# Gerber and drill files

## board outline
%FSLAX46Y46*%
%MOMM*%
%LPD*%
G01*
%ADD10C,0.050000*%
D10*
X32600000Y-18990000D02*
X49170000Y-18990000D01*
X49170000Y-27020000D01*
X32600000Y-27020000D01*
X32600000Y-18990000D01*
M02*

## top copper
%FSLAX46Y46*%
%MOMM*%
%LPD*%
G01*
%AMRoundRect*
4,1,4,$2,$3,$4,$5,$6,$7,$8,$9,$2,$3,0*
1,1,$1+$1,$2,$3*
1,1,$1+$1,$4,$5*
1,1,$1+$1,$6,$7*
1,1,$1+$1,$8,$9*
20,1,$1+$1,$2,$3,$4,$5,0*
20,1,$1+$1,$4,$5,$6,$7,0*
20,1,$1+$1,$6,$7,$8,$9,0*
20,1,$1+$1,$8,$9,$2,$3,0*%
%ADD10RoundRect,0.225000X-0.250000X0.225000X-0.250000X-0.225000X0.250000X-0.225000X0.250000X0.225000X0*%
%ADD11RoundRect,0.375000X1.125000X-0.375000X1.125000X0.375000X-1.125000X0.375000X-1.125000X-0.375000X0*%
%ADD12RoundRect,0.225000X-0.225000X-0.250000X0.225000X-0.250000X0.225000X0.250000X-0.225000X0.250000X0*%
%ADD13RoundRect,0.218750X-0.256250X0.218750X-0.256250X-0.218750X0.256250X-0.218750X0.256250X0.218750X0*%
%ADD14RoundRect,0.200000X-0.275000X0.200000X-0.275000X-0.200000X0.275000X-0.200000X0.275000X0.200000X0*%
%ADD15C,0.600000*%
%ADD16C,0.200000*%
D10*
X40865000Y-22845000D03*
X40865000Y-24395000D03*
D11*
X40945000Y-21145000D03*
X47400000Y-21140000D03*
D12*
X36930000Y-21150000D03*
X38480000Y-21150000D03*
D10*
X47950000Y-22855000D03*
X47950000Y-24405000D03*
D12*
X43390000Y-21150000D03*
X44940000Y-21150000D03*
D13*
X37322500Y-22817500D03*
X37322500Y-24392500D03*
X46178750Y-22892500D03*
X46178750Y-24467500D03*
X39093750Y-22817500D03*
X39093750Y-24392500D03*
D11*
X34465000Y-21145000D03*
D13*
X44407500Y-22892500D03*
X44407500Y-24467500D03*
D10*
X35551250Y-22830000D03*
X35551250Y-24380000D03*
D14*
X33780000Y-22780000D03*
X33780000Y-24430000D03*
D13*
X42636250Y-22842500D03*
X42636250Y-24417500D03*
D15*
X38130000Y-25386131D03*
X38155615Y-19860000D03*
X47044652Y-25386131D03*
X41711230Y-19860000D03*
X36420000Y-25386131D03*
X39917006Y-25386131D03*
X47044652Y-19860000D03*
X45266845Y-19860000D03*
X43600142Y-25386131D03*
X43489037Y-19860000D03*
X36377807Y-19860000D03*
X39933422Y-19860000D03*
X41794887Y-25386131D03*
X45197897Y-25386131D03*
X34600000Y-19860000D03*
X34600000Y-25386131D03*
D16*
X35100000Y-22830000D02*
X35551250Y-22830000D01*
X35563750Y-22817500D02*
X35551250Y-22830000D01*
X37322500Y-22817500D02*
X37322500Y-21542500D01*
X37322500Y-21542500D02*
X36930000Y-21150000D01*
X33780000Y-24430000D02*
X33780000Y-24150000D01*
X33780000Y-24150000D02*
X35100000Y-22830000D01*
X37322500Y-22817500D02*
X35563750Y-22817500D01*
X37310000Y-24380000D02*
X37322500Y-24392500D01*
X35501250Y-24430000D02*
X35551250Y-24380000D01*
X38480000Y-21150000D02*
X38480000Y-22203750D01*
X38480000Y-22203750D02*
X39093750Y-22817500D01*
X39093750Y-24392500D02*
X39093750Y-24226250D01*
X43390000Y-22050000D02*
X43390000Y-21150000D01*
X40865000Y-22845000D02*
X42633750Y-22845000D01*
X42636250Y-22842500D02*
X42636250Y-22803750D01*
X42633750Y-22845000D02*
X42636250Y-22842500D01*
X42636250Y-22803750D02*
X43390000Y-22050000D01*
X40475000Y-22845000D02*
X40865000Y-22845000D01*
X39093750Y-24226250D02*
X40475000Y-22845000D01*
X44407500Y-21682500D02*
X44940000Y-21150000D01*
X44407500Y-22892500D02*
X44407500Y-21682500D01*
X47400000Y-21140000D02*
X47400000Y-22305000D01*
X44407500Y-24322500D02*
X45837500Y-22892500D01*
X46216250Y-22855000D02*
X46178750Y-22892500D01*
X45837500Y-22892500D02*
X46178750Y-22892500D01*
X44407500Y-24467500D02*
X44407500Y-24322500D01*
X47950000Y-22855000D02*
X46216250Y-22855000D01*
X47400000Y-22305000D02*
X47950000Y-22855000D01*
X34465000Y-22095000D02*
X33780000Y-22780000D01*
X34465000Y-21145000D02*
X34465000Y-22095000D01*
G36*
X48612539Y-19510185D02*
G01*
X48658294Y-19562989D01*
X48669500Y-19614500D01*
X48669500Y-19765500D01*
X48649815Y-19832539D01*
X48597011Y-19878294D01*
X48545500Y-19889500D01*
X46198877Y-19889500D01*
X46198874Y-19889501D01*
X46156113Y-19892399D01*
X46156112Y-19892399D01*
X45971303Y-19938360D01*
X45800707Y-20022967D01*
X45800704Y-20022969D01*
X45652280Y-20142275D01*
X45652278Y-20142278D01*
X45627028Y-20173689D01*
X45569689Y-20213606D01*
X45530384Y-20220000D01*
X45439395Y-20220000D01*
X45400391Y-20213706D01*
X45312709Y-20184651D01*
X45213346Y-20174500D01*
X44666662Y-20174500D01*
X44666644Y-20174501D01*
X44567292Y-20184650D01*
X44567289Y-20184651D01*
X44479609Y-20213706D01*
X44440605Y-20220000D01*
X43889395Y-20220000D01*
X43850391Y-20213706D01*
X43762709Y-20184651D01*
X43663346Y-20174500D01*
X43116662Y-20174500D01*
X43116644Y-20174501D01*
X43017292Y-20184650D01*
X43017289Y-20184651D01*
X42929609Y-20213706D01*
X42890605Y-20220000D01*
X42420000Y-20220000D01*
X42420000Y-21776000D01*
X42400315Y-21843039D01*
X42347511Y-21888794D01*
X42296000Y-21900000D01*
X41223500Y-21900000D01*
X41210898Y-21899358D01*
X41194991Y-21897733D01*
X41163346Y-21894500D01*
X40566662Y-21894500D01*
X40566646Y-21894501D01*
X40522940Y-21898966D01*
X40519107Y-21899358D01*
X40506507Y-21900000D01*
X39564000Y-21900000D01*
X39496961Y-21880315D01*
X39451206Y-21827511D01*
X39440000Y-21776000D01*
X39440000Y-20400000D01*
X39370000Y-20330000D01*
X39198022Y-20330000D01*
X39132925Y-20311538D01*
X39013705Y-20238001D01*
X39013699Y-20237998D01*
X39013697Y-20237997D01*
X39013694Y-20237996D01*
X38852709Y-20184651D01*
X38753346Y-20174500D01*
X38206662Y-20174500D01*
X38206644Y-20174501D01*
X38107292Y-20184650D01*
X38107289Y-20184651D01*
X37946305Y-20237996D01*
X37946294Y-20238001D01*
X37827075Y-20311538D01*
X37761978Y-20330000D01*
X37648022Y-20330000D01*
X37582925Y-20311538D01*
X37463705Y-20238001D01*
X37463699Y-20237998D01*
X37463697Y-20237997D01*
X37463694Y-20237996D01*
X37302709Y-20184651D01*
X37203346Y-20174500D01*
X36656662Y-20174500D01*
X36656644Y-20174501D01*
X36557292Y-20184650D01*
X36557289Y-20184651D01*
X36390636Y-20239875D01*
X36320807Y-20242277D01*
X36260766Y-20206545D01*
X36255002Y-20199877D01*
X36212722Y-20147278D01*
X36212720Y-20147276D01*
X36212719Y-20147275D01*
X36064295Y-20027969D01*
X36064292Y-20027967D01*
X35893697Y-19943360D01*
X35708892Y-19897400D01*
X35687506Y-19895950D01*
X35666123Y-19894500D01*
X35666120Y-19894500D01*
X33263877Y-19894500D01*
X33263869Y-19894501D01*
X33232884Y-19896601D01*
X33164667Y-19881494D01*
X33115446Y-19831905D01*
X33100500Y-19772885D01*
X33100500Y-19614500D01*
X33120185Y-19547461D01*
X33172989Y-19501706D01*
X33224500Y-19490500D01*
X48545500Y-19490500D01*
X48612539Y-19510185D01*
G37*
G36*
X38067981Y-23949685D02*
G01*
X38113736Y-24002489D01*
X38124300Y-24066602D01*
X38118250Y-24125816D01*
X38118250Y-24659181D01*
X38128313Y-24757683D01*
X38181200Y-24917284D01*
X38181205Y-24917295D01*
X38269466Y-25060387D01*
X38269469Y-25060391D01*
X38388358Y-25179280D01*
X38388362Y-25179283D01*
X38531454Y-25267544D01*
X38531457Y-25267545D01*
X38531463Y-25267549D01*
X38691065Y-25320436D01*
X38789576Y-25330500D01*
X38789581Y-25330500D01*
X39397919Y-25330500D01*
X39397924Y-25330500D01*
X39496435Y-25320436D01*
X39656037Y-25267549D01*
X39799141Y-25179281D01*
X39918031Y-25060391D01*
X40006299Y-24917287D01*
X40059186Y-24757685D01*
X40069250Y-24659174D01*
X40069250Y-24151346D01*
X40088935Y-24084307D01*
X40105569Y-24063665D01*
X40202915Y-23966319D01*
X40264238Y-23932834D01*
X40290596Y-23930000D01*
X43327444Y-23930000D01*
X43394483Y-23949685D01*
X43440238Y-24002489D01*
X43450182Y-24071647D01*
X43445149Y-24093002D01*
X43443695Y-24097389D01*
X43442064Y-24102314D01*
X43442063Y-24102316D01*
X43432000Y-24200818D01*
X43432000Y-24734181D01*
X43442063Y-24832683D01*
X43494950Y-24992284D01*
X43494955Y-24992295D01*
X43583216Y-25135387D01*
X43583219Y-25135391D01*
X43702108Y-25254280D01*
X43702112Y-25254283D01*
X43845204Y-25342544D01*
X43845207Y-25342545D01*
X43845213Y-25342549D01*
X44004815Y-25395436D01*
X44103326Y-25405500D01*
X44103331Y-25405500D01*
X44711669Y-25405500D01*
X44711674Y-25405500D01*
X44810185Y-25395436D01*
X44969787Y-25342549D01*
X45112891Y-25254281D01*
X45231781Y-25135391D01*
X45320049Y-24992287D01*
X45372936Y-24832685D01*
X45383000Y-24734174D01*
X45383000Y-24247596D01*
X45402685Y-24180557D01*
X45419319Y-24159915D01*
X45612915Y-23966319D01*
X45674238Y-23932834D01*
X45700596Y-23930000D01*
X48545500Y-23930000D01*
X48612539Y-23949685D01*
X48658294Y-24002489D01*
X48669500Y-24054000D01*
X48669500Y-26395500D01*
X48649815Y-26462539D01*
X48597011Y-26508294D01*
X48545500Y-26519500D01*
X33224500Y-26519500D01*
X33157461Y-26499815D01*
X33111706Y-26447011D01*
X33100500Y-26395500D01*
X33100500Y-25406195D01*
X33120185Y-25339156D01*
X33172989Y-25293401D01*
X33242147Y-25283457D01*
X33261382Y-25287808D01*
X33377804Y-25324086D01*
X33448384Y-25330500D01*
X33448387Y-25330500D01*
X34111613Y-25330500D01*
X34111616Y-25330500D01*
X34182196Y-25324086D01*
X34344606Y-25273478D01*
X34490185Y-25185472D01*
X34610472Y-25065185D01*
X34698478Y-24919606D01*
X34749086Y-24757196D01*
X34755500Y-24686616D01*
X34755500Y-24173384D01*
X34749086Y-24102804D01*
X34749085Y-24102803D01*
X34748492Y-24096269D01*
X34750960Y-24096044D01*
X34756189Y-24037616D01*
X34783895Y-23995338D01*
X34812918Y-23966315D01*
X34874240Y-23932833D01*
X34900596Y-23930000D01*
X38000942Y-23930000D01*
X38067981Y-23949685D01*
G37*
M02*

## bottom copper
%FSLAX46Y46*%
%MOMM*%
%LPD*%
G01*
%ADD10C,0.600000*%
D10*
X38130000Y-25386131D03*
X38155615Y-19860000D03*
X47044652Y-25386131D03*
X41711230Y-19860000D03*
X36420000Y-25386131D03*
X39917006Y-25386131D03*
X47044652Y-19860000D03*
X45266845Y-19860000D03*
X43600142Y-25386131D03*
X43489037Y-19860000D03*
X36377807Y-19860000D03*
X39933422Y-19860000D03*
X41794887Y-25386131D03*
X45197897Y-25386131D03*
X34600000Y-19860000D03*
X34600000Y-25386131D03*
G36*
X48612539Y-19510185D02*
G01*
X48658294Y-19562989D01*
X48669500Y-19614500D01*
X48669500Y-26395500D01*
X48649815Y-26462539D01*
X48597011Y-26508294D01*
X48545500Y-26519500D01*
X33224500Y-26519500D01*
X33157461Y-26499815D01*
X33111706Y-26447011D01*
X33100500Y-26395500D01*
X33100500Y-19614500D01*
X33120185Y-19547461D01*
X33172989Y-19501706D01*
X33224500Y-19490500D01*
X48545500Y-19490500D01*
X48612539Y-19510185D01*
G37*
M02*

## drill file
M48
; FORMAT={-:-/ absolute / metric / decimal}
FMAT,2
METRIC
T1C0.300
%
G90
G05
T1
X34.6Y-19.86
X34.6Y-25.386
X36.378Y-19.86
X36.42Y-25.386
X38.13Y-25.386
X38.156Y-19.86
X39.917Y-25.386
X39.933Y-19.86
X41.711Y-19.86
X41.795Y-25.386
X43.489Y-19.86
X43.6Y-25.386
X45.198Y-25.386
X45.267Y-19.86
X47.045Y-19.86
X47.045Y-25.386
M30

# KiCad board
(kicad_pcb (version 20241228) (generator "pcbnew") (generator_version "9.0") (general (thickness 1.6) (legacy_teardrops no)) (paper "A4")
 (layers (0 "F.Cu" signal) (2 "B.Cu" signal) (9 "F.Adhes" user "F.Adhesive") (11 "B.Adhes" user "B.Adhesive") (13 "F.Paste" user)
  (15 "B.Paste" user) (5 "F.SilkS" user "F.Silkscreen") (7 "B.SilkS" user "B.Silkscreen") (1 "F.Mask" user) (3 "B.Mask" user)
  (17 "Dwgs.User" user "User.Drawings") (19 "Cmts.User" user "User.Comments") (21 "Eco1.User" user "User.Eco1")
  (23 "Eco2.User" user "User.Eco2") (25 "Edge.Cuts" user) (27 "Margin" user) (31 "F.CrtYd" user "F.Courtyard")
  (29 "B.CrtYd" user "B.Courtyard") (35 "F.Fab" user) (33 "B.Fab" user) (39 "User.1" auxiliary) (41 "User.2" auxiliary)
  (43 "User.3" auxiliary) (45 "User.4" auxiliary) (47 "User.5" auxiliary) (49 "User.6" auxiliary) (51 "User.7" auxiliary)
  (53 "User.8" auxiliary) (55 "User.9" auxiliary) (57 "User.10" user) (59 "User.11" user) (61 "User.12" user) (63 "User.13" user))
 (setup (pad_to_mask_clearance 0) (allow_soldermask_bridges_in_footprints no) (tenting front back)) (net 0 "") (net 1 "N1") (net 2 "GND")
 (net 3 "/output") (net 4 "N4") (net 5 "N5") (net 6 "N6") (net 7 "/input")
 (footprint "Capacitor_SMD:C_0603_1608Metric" (layer "F.Cu") (at 40.865 23.62 -90)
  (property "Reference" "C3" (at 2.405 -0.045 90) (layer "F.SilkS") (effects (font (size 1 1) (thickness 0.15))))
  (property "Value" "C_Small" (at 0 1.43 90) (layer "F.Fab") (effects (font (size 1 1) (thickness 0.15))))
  (pad "1" smd roundrect (at -0.775 0 270) (size 0.9 0.95) (layers "F.Cu" "F.Mask" "F.Paste") (roundrect_rratio 0.25) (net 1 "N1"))
  (pad "2" smd roundrect (at 0.775 0 270) (size 0.9 0.95) (layers "F.Cu" "F.Mask" "F.Paste") (roundrect_rratio 0.25) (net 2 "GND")))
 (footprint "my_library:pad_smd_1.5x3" (layer "F.Cu") (at 40.945 21.145)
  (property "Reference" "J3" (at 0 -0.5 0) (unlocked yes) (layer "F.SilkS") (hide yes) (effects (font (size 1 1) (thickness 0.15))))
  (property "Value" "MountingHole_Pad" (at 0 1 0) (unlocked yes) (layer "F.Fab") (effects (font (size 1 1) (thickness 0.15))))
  (pad "1" smd roundrect (at 0 0 90) (size 1.5 3) (layers "F.Cu" "F.Mask" "F.Paste") (roundrect_rratio 0.25) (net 2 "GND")
   (thermal_bridge_angle 45)))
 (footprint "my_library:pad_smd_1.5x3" (layer "F.Cu") (at 47.4 21.14)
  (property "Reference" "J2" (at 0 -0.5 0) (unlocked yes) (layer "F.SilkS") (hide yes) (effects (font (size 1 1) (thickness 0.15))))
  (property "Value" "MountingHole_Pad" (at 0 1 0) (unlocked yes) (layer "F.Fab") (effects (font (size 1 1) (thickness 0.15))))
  (pad "1" smd roundrect (at 0 0 90) (size 1.5 3) (layers "F.Cu" "F.Mask" "F.Paste") (roundrect_rratio 0.25) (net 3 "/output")
   (thermal_bridge_angle 45)))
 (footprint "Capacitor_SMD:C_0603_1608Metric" (layer "F.Cu") (at 37.705 21.15)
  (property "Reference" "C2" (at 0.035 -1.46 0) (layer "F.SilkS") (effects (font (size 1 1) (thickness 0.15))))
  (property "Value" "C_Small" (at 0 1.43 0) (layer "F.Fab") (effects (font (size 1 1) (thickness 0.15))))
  (pad "1" smd roundrect (at -0.775 0) (size 0.9 0.95) (layers "F.Cu" "F.Mask" "F.Paste") (roundrect_rratio 0.25) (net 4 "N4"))
  (pad "2" smd roundrect (at 0.775 0) (size 0.9 0.95) (layers "F.Cu" "F.Mask" "F.Paste") (roundrect_rratio 0.25) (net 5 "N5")))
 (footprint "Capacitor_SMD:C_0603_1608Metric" (layer "F.Cu") (at 47.95 23.63 -90)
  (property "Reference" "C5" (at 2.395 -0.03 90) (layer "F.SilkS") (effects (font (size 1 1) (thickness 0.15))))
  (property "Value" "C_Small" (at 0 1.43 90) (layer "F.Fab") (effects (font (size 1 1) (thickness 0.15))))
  (pad "1" smd roundrect (at -0.775 0 270) (size 0.9 0.95) (layers "F.Cu" "F.Mask" "F.Paste") (roundrect_rratio 0.25) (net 3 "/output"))
  (pad "2" smd roundrect (at 0.775 0 270) (size 0.9 0.95) (layers "F.Cu" "F.Mask" "F.Paste") (roundrect_rratio 0.25) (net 2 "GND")))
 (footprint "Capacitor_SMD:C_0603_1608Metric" (layer "F.Cu") (at 44.165 21.15)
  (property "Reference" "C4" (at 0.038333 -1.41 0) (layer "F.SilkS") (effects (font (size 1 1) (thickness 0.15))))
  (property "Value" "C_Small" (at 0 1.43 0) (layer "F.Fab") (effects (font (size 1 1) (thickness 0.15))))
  (pad "1" smd roundrect (at -0.775 0) (size 0.9 0.95) (layers "F.Cu" "F.Mask" "F.Paste") (roundrect_rratio 0.25) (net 1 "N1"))
  (pad "2" smd roundrect (at 0.775 0) (size 0.9 0.95) (layers "F.Cu" "F.Mask" "F.Paste") (roundrect_rratio 0.25) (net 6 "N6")))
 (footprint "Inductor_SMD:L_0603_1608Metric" (layer "F.Cu") (at 37.3225 23.605 -90)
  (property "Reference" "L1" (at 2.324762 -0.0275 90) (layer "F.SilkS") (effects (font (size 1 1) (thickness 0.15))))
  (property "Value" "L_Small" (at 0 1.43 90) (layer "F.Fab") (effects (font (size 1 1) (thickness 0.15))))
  (pad "1" smd roundrect (at -0.7875 0 270) (size 0.875 0.95) (layers "F.Cu" "F.Mask" "F.Paste") (roundrect_rratio 0.25) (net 4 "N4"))
  (pad "2" smd roundrect (at 0.7875 0 270) (size 0.875 0.95) (layers "F.Cu" "F.Mask" "F.Paste") (roundrect_rratio 0.25) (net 2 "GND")))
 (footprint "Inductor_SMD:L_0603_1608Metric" (layer "F.Cu") (at 46.17875 23.68 -90)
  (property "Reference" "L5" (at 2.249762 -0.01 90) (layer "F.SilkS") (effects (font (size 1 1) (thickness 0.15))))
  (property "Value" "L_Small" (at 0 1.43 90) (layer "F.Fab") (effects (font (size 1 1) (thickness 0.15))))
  (pad "1" smd roundrect (at -0.7875 0 270) (size 0.875 0.95) (layers "F.Cu" "F.Mask" "F.Paste") (roundrect_rratio 0.25) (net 3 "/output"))
  (pad "2" smd roundrect (at 0.7875 0 270) (size 0.875 0.95) (layers "F.Cu" "F.Mask" "F.Paste") (roundrect_rratio 0.25) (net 2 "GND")))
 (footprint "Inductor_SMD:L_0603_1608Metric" (layer "F.Cu") (at 39.09375 23.605 -90)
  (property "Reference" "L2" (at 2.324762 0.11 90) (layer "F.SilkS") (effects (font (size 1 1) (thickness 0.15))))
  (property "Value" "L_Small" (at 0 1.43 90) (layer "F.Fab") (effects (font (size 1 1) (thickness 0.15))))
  (pad "1" smd roundrect (at -0.7875 0 270) (size 0.875 0.95) (layers "F.Cu" "F.Mask" "F.Paste") (roundrect_rratio 0.25) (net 5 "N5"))
  (pad "2" smd roundrect (at 0.7875 0 270) (size 0.875 0.95) (layers "F.Cu" "F.Mask" "F.Paste") (roundrect_rratio 0.25) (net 1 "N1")))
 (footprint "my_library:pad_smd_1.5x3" (layer "F.Cu") (at 34.465 21.145)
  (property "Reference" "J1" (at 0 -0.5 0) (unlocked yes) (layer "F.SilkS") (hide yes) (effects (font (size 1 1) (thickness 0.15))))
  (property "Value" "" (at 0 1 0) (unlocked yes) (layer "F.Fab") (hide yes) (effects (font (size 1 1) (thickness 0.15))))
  (pad "1" smd roundrect (at 0 0 90) (size 1.5 3) (layers "F.Cu" "F.Mask" "F.Paste") (roundrect_rratio 0.25) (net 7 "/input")
   (thermal_bridge_angle 45)))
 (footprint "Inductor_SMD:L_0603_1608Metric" (layer "F.Cu") (at 44.4075 23.68 -90)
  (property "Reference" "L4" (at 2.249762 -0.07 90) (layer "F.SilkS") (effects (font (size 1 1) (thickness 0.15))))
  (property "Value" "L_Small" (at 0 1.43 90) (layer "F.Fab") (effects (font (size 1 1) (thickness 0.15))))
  (pad "1" smd roundrect (at -0.7875 0 270) (size 0.875 0.95) (layers "F.Cu" "F.Mask" "F.Paste") (roundrect_rratio 0.25) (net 6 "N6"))
  (pad "2" smd roundrect (at 0.7875 0 270) (size 0.875 0.95) (layers "F.Cu" "F.Mask" "F.Paste") (roundrect_rratio 0.25) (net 3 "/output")))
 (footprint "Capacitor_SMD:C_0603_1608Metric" (layer "F.Cu") (at 35.55125 23.605 -90)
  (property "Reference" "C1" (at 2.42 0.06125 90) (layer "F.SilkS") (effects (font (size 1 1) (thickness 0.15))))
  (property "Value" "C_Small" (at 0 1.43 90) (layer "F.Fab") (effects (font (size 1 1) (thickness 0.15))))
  (pad "1" smd roundrect (at -0.775 0 270) (size 0.9 0.95) (layers "F.Cu" "F.Mask" "F.Paste") (roundrect_rratio 0.25) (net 4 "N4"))
  (pad "2" smd roundrect (at 0.775 0 270) (size 0.9 0.95) (layers "F.Cu" "F.Mask" "F.Paste") (roundrect_rratio 0.25) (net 2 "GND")))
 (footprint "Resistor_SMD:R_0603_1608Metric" (layer "F.Cu") (at 33.78 23.605 -90)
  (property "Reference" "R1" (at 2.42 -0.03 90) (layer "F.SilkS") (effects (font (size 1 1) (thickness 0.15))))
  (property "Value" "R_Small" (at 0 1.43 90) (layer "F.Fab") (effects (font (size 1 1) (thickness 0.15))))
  (pad "1" smd roundrect (at -0.825 0 270) (size 0.8 0.95) (layers "F.Cu" "F.Mask" "F.Paste") (roundrect_rratio 0.25) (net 7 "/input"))
  (pad "2" smd roundrect (at 0.825 0 270) (size 0.8 0.95) (layers "F.Cu" "F.Mask" "F.Paste") (roundrect_rratio 0.25) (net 4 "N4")))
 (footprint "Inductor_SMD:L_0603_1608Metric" (layer "F.Cu") (at 42.63625 23.63 -90)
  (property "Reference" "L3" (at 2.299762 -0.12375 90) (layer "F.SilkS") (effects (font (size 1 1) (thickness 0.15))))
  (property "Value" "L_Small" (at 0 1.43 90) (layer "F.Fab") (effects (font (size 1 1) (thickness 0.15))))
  (pad "1" smd roundrect (at -0.7875 0 270) (size 0.875 0.95) (layers "F.Cu" "F.Mask" "F.Paste") (roundrect_rratio 0.25) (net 1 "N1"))
  (pad "2" smd roundrect (at 0.7875 0 270) (size 0.875 0.95) (layers "F.Cu" "F.Mask" "F.Paste") (roundrect_rratio 0.25) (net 2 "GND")))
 (gr_rect (start 32.6 18.99) (end 49.17 27.02) (stroke (width 0.05) (type default)) (fill no) (layer "Edge.Cuts"))
 (segment (start 35.1 22.83) (end 35.55125 22.83) (width 0.2) (layer "F.Cu") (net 4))
 (segment (start 35.56375 22.8175) (end 35.55125 22.83) (width 0.2) (layer "F.Cu") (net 4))
 (segment (start 37.3225 22.8175) (end 37.3225 21.5425) (width 0.2) (layer "F.Cu") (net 4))
 (segment (start 37.3225 21.5425) (end 36.93 21.15) (width 0.2) (layer "F.Cu") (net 4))
 (segment (start 33.78 24.43) (end 33.78 24.15) (width 0.2) (layer "F.Cu") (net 4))
 (segment (start 33.78 24.15) (end 35.1 22.83) (width 0.2) (layer "F.Cu") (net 4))
 (segment (start 37.3225 22.8175) (end 35.56375 22.8175) (width 0.2) (layer "F.Cu") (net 4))
 (segment (start 37.31 24.38) (end 37.3225 24.3925) (width 0.2) (layer "F.Cu") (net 2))
 (segment (start 35.50125 24.43) (end 35.55125 24.38) (width 0.2) (layer "F.Cu") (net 2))
 (via (at 38.13 25.386131) (size 0.6) (drill 0.3) (layers "F.Cu" "B.Cu") (free yes) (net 2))
 (via (at 38.155615 19.86) (size 0.6) (drill 0.3) (layers "F.Cu" "B.Cu") (free yes) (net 2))
 (via (at 47.044652 25.386131) (size 0.6) (drill 0.3) (layers "F.Cu" "B.Cu") (free yes) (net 2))
 (via (at 41.71123 19.86) (size 0.6) (drill 0.3) (layers "F.Cu" "B.Cu") (free yes) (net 2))
 (via (at 36.42 25.386131) (size 0.6) (drill 0.3) (layers "F.Cu" "B.Cu") (free yes) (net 2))
 (via (at 39.917006 25.386131) (size 0.6) (drill 0.3) (layers "F.Cu" "B.Cu") (free yes) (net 2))
 (via (at 47.044652 19.86) (size 0.6) (drill 0.3) (layers "F.Cu" "B.Cu") (free yes) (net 2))
 (via (at 45.266845 19.86) (size 0.6) (drill 0.3) (layers "F.Cu" "B.Cu") (free yes) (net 2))
 (via (at 43.600142 25.386131) (size 0.6) (drill 0.3) (layers "F.Cu" "B.Cu") (free yes) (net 2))
 (via (at 43.489037 19.86) (size 0.6) (drill 0.3) (layers "F.Cu" "B.Cu") (free yes) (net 2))
 (via (at 36.377807 19.86) (size 0.6) (drill 0.3) (layers "F.Cu" "B.Cu") (free yes) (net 2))
 (via (at 39.933422 19.86) (size 0.6) (drill 0.3) (layers "F.Cu" "B.Cu") (free yes) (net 2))
 (via (at 41.794887 25.386131) (size 0.6) (drill 0.3) (layers "F.Cu" "B.Cu") (free yes) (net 2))
 (via (at 45.197897 25.386131) (size 0.6) (drill 0.3) (layers "F.Cu" "B.Cu") (free yes) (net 2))
 (via (at 34.6 19.86) (size 0.6) (drill 0.3) (layers "F.Cu" "B.Cu") (free yes) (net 2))
 (via (at 34.6 25.386131) (size 0.6) (drill 0.3) (layers "F.Cu" "B.Cu") (free yes) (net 2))
 (segment (start 38.48 21.15) (end 38.48 22.20375) (width 0.2) (layer "F.Cu") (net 5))
 (segment (start 38.48 22.20375) (end 39.09375 22.8175) (width 0.2) (layer "F.Cu") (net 5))
 (segment (start 39.09375 24.3925) (end 39.09375 24.22625) (width 0.2) (layer "F.Cu") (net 1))
 (segment (start 43.39 22.05) (end 43.39 21.15) (width 0.2) (layer "F.Cu") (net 1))
 (segment (start 40.865 22.845) (end 42.63375 22.845) (width 0.2) (layer "F.Cu") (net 1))
 (segment (start 42.63625 22.8425) (end 42.63625 22.80375) (width 0.2) (layer "F.Cu") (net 1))
 (segment (start 42.63375 22.845) (end 42.63625 22.8425) (width 0.2) (layer "F.Cu") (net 1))
 (segment (start 42.63625 22.80375) (end 43.39 22.05) (width 0.2) (layer "F.Cu") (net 1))
 (segment (start 40.475 22.845) (end 40.865 22.845) (width 0.2) (layer "F.Cu") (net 1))
 (segment (start 39.09375 24.22625) (end 40.475 22.845) (width 0.2) (layer "F.Cu") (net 1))
 (segment (start 44.4075 21.6825) (end 44.94 21.15) (width 0.2) (layer "F.Cu") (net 6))
 (segment (start 44.4075 22.8925) (end 44.4075 21.6825) (width 0.2) (layer "F.Cu") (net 6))
 (segment (start 47.4 21.14) (end 47.4 22.305) (width 0.2) (layer "F.Cu") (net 3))
 (segment (start 44.4075 24.3225) (end 45.8375 22.8925) (width 0.2) (layer "F.Cu") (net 3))
 (segment (start 46.21625 22.855) (end 46.17875 22.8925) (width 0.2) (layer "F.Cu") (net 3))
 (segment (start 45.8375 22.8925) (end 46.17875 22.8925) (width 0.2) (layer "F.Cu") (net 3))
 (segment (start 44.4075 24.4675) (end 44.4075 24.3225) (width 0.2) (layer "F.Cu") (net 3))
 (segment (start 47.95 22.855) (end 46.21625 22.855) (width 0.2) (layer "F.Cu") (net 3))
 (segment (start 47.4 22.305) (end 47.95 22.855) (width 0.2) (layer "F.Cu") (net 3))
 (segment (start 34.465 22.095) (end 33.78 22.78) (width 0.2) (layer "F.Cu") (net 7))
 (segment (start 34.465 21.145) (end 34.465 22.095) (width 0.2) (layer "F.Cu") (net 7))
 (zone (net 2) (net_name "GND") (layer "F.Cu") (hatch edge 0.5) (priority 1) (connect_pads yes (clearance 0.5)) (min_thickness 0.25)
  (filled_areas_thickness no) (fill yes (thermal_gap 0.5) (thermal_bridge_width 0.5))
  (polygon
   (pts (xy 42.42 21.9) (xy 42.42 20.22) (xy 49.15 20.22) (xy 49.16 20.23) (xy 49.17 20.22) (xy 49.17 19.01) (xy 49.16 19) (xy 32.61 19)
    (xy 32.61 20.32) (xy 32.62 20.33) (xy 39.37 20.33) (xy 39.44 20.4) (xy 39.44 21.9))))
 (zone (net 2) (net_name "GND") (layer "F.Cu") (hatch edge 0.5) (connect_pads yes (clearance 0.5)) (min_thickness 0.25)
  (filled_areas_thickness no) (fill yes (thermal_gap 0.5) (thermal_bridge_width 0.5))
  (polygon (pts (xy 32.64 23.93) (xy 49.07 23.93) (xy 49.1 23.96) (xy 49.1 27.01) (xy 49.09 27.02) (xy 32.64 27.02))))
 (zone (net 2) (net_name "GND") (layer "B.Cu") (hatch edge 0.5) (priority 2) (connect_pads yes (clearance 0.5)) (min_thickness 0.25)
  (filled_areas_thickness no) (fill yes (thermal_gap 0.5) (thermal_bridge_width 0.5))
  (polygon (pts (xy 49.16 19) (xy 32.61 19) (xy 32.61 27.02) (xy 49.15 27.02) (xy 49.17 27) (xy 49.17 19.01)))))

